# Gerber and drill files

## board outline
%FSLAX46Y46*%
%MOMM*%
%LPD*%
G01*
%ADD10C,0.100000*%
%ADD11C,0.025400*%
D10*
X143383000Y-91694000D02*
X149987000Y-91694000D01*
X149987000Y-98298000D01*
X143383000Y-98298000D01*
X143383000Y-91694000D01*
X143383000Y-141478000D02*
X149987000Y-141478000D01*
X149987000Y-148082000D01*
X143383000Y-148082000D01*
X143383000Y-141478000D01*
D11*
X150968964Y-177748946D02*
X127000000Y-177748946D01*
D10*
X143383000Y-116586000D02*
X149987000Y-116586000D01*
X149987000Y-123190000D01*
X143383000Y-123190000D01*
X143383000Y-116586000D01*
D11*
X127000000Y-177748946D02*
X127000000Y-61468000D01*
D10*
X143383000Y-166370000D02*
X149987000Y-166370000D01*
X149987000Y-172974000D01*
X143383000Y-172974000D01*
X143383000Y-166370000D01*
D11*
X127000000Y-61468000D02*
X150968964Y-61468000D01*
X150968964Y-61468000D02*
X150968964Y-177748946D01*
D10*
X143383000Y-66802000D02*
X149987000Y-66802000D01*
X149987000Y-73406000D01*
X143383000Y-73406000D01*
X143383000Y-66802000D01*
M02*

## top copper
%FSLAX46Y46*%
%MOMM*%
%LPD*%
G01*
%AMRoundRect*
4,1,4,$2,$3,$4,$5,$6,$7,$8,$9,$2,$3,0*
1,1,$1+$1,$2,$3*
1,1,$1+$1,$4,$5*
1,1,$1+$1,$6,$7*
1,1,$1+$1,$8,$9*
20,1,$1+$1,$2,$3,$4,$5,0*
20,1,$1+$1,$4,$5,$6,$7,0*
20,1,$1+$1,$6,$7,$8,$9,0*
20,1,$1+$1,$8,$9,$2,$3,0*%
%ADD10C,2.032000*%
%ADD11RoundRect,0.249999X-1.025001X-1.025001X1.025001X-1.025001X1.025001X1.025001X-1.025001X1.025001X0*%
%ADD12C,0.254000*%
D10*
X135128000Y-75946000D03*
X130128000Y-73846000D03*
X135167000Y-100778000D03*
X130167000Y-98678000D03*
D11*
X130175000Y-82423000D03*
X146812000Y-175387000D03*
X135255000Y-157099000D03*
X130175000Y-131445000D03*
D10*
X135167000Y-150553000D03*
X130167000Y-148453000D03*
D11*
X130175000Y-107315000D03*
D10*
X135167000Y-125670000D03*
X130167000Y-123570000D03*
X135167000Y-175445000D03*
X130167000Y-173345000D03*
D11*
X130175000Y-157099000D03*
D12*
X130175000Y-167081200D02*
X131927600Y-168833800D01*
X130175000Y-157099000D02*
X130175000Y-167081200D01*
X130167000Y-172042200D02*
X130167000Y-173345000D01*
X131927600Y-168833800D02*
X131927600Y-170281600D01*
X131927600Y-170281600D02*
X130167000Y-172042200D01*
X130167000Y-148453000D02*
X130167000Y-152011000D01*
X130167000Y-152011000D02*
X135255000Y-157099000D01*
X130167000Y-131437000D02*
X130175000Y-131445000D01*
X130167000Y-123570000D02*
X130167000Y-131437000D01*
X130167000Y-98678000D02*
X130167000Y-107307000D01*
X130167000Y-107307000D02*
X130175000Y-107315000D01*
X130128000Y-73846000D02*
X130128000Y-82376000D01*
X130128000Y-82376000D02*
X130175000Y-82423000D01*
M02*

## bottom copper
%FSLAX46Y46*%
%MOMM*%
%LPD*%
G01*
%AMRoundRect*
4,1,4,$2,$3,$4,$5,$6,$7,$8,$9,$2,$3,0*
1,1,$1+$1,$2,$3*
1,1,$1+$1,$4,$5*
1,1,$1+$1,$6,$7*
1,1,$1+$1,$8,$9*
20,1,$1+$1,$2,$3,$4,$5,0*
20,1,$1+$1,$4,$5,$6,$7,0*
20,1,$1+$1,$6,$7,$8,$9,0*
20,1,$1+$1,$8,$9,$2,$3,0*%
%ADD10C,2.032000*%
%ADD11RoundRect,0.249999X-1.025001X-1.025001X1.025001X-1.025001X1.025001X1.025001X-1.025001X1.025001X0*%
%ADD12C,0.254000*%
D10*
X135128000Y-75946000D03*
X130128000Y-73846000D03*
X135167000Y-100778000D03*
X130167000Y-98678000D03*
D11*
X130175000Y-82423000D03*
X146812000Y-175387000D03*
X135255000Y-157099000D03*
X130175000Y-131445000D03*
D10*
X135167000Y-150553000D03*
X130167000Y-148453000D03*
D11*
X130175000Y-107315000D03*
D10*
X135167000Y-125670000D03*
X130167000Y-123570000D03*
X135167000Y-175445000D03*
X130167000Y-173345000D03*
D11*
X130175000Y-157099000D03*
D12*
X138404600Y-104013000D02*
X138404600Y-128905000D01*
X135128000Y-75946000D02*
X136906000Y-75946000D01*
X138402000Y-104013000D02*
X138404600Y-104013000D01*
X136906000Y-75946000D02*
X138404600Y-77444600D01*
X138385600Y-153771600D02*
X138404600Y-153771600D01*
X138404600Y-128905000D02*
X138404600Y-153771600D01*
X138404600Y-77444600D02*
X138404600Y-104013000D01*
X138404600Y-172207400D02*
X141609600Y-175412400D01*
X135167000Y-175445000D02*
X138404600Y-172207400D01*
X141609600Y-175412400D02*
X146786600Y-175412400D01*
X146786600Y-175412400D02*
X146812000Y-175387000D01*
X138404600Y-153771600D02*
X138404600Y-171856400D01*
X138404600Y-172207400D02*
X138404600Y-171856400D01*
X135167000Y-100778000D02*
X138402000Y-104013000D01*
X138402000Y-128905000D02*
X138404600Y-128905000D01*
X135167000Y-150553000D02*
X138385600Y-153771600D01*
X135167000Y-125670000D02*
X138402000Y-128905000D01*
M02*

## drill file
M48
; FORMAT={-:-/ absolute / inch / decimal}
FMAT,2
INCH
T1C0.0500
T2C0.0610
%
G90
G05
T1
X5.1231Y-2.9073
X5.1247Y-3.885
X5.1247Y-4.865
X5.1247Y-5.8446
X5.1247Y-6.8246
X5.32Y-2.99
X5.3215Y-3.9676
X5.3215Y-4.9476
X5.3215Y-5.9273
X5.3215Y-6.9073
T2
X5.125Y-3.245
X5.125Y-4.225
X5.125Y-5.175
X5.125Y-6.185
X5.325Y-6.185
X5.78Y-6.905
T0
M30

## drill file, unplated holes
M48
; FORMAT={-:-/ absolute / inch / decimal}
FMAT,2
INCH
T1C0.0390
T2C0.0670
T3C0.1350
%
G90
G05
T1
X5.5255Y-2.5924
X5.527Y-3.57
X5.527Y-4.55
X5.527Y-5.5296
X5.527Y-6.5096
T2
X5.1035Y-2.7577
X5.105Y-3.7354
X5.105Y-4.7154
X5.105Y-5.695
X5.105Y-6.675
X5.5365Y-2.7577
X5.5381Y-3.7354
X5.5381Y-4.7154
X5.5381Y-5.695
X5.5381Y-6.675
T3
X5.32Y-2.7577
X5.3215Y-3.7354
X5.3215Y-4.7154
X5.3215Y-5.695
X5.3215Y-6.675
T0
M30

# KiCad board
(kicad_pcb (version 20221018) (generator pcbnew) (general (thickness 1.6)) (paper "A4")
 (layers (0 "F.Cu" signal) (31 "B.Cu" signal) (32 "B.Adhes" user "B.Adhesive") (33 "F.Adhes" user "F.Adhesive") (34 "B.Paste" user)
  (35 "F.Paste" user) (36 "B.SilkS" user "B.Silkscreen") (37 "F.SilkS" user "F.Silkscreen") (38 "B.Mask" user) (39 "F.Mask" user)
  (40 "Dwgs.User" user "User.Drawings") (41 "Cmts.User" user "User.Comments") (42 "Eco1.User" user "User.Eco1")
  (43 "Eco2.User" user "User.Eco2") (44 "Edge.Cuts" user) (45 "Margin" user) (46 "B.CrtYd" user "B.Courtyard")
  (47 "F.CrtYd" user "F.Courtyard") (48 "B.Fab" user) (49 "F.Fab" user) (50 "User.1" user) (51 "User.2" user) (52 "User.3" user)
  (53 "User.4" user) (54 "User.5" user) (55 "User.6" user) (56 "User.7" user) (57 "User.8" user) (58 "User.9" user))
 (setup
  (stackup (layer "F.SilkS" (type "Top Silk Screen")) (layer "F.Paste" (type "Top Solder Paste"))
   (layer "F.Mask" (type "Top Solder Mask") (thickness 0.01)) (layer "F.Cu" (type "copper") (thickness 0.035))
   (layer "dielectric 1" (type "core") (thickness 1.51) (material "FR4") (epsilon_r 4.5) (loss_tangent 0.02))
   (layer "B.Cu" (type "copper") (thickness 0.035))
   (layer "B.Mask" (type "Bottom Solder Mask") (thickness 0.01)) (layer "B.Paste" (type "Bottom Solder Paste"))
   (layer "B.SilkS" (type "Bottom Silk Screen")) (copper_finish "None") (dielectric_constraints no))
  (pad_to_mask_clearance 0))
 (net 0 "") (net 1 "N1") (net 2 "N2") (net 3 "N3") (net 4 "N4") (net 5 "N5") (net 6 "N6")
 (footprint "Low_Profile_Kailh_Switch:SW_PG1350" (layer "F.Cu") (at 135.128 70.046)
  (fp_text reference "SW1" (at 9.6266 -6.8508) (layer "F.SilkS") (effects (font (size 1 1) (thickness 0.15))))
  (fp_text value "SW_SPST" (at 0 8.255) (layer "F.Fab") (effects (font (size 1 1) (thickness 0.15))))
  (pad "" np_thru_hole circle (at -5.5 0) (size 1.7018 1.7018) (drill 1.7018) (layers "*.Cu" "*.Mask"))
  (pad "" np_thru_hole circle (at 0 0) (size 3.429 3.429) (drill 3.429) (layers "*.Cu" "*.Mask"))
  (pad "" np_thru_hole circle (at 5.22 -4.2) (size 0.9906 0.9906) (drill 0.9906) (layers "*.Cu" "*.Mask"))
  (pad "" np_thru_hole circle (at 5.5 0) (size 1.7018 1.7018) (drill 1.7018) (layers "*.Cu" "*.Mask"))
  (pad "1" thru_hole circle (at 0 5.9) (size 2.032 2.032) (drill 1.27) (layers "*.Cu" "*.Mask") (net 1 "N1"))
  (pad "2" thru_hole circle (at -5 3.8) (size 2.032 2.032) (drill 1.27) (layers "*.Cu" "*.Mask") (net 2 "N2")))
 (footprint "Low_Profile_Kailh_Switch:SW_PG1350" (layer "F.Cu") (at 135.167 94.878)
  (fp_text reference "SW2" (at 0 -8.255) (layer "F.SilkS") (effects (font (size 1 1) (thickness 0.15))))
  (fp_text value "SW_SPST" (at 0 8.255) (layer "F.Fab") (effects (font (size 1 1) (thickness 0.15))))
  (pad "" np_thru_hole circle (at -5.5 0) (size 1.7018 1.7018) (drill 1.7018) (layers "*.Cu" "*.Mask"))
  (pad "" np_thru_hole circle (at 0 0) (size 3.429 3.429) (drill 3.429) (layers "*.Cu" "*.Mask"))
  (pad "" np_thru_hole circle (at 5.22 -4.2) (size 0.9906 0.9906) (drill 0.9906) (layers "*.Cu" "*.Mask"))
  (pad "" np_thru_hole circle (at 5.5 0) (size 1.7018 1.7018) (drill 1.7018) (layers "*.Cu" "*.Mask"))
  (pad "1" thru_hole circle (at 0 5.9) (size 2.032 2.032) (drill 1.27) (layers "*.Cu" "*.Mask") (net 1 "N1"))
  (pad "2" thru_hole circle (at -5 3.8) (size 2.032 2.032) (drill 1.27) (layers "*.Cu" "*.Mask") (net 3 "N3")))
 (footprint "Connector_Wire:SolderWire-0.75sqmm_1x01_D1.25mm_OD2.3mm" (layer "F.Cu") (at 130.175 82.423)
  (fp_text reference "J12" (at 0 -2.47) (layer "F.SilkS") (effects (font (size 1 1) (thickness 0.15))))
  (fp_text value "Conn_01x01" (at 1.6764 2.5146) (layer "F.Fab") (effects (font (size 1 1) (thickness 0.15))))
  (pad "1" thru_hole roundrect (at 0 0) (size 2.55 2.55) (drill 1.55) (layers "*.Cu" "*.Mask") (roundrect_rratio 0.09803882353) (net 2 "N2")))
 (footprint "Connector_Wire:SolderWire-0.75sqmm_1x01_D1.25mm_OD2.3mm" (layer "F.Cu") (at 146.812 175.387)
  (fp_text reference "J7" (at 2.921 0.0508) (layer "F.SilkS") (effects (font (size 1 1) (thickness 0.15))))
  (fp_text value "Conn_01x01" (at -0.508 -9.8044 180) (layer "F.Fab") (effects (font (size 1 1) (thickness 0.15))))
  (pad "1" thru_hole roundrect (at 0 0) (size 2.55 2.55) (drill 1.55) (layers "*.Cu" "*.Mask") (roundrect_rratio 0.09803882353) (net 1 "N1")))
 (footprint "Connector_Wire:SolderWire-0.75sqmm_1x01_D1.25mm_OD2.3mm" (layer "F.Cu") (at 135.255 157.099)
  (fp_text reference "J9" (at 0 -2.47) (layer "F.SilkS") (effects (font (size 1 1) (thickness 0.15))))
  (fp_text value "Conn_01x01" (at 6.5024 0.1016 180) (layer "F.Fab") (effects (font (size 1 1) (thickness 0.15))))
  (pad "1" thru_hole roundrect (at 0 0) (size 2.55 2.55) (drill 1.55) (layers "*.Cu" "*.Mask") (roundrect_rratio 0.09803882353) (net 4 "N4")))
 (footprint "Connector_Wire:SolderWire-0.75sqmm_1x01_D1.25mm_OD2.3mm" (layer "F.Cu") (at 130.175 131.445)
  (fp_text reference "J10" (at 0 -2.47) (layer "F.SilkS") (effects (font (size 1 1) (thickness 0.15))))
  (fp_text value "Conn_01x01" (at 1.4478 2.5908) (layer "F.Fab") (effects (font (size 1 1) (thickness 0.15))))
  (pad "1" thru_hole roundrect (at 0 0) (size 2.55 2.55) (drill 1.55) (layers "*.Cu" "*.Mask") (roundrect_rratio 0.09803882353) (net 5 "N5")))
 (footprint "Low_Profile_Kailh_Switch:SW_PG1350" (layer "F.Cu") (at 135.167 144.653)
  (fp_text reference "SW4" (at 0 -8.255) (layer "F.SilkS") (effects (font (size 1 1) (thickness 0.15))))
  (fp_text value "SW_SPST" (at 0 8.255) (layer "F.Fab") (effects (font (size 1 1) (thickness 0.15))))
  (pad "" np_thru_hole circle (at -5.5 0) (size 1.7018 1.7018) (drill 1.7018) (layers "*.Cu" "*.Mask"))
  (pad "" np_thru_hole circle (at 0 0) (size 3.429 3.429) (drill 3.429) (layers "*.Cu" "*.Mask"))
  (pad "" np_thru_hole circle (at 5.22 -4.2) (size 0.9906 0.9906) (drill 0.9906) (layers "*.Cu" "*.Mask"))
  (pad "" np_thru_hole circle (at 5.5 0) (size 1.7018 1.7018) (drill 1.7018) (layers "*.Cu" "*.Mask"))
  (pad "1" thru_hole circle (at 0 5.9) (size 2.032 2.032) (drill 1.27) (layers "*.Cu" "*.Mask") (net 1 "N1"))
  (pad "2" thru_hole circle (at -5 3.8) (size 2.032 2.032) (drill 1.27) (layers "*.Cu" "*.Mask") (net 4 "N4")))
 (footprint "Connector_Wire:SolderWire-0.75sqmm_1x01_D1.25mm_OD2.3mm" (layer "F.Cu") (at 130.175 107.315)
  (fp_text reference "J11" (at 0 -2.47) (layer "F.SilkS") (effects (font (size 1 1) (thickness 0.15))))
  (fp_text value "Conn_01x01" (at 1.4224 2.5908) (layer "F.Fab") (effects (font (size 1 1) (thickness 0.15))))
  (pad "1" thru_hole roundrect (at 0 0) (size 2.55 2.55) (drill 1.55) (layers "*.Cu" "*.Mask") (roundrect_rratio 0.09803882353) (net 3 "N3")))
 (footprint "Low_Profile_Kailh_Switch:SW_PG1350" (layer "F.Cu") (at 135.167 119.77)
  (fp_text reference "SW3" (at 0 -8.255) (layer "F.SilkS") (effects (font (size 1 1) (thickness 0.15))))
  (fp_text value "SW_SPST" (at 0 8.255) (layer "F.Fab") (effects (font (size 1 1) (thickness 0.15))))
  (pad "" np_thru_hole circle (at -5.5 0) (size 1.7018 1.7018) (drill 1.7018) (layers "*.Cu" "*.Mask"))
  (pad "" np_thru_hole circle (at 0 0) (size 3.429 3.429) (drill 3.429) (layers "*.Cu" "*.Mask"))
  (pad "" np_thru_hole circle (at 5.22 -4.2) (size 0.9906 0.9906) (drill 0.9906) (layers "*.Cu" "*.Mask"))
  (pad "" np_thru_hole circle (at 5.5 0) (size 1.7018 1.7018) (drill 1.7018) (layers "*.Cu" "*.Mask"))
  (pad "1" thru_hole circle (at 0 5.9) (size 2.032 2.032) (drill 1.27) (layers "*.Cu" "*.Mask") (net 1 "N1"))
  (pad "2" thru_hole circle (at -5 3.8) (size 2.032 2.032) (drill 1.27) (layers "*.Cu" "*.Mask") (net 5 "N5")))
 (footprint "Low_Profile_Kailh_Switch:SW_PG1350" (layer "F.Cu") (at 135.167 169.545)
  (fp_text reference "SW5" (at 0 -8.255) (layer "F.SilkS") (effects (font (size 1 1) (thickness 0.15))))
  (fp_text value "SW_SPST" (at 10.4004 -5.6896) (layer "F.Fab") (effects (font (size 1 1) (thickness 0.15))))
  (pad "" np_thru_hole circle (at -5.5 0) (size 1.7018 1.7018) (drill 1.7018) (layers "*.Cu" "*.Mask"))
  (pad "" np_thru_hole circle (at 0 0) (size 3.429 3.429) (drill 3.429) (layers "*.Cu" "*.Mask"))
  (pad "" np_thru_hole circle (at 5.22 -4.2) (size 0.9906 0.9906) (drill 0.9906) (layers "*.Cu" "*.Mask"))
  (pad "" np_thru_hole circle (at 5.5 0) (size 1.7018 1.7018) (drill 1.7018) (layers "*.Cu" "*.Mask"))
  (pad "1" thru_hole circle (at 0 5.9) (size 2.032 2.032) (drill 1.27) (layers "*.Cu" "*.Mask") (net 1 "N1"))
  (pad "2" thru_hole circle (at -5 3.8) (size 2.032 2.032) (drill 1.27) (layers "*.Cu" "*.Mask") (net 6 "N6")))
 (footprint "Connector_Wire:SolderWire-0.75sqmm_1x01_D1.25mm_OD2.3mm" (layer "F.Cu") (at 130.175 157.099)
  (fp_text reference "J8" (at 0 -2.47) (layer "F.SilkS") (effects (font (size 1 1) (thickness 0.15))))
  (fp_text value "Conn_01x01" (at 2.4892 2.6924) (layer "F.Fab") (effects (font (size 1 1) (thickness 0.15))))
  (pad "1" thru_hole roundrect (at 0 0) (size 2.55 2.55) (drill 1.55) (layers "*.Cu" "*.Mask") (roundrect_rratio 0.09803882353) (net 6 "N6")))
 (gr_rect (start 143.383 91.694) (end 149.987 98.298) (stroke (width 0.1) (type default)) (fill none) (layer "Edge.Cuts"))
 (gr_rect (start 143.383 141.478) (end 149.987 148.082) (stroke (width 0.1) (type default)) (fill none) (layer "Edge.Cuts"))
 (gr_line (start 150.968964 177.748946) (end 127 177.748946) (stroke (width 0.0254) (type default)) (layer "Edge.Cuts"))
 (gr_rect (start 143.383 116.586) (end 149.987 123.19) (stroke (width 0.1) (type default)) (fill none) (layer "Edge.Cuts"))
 (gr_line (start 127 177.748946) (end 127 61.468) (stroke (width 0.0254) (type default)) (layer "Edge.Cuts"))
 (gr_rect (start 143.383 166.37) (end 149.987 172.974) (stroke (width 0.1) (type default)) (fill none) (layer "Edge.Cuts"))
 (gr_line (start 127 61.468) (end 150.968964 61.468) (stroke (width 0.0254) (type default)) (layer "Edge.Cuts"))
 (gr_line (start 150.968964 61.468) (end 150.968964 177.748946) (stroke (width 0.0254) (type default)) (layer "Edge.Cuts"))
 (gr_rect (start 143.383 66.802) (end 149.987 73.406) (stroke (width 0.1) (type default)) (fill none) (layer "Edge.Cuts"))
 (segment (start 138.4046 104.013) (end 138.4046 128.905) (width 0.254) (layer "B.Cu") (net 1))
 (segment (start 135.128 75.946) (end 136.906 75.946) (width 0.254) (layer "B.Cu") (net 1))
 (segment (start 138.402 104.013) (end 138.4046 104.013) (width 0.254) (layer "B.Cu") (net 1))
 (segment (start 136.906 75.946) (end 138.4046 77.4446) (width 0.254) (layer "B.Cu") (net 1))
 (segment (start 138.3856 153.7716) (end 138.4046 153.7716) (width 0.254) (layer "B.Cu") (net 1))
 (segment (start 138.4046 128.905) (end 138.4046 153.7716) (width 0.254) (layer "B.Cu") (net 1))
 (segment (start 138.4046 77.4446) (end 138.4046 104.013) (width 0.254) (layer "B.Cu") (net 1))
 (segment (start 138.4046 172.2074) (end 141.6096 175.4124) (width 0.254) (layer "B.Cu") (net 1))
 (segment (start 135.167 175.445) (end 138.4046 172.2074) (width 0.254) (layer "B.Cu") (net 1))
 (segment (start 141.6096 175.4124) (end 146.7866 175.4124) (width 0.254) (layer "B.Cu") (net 1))
 (segment (start 146.7866 175.4124) (end 146.812 175.387) (width 0.254) (layer "B.Cu") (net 1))
 (segment (start 138.4046 153.7716) (end 138.4046 171.8564) (width 0.254) (layer "B.Cu") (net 1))
 (segment (start 138.4046 172.2074) (end 138.4046 171.8564) (width 0.254) (layer "B.Cu") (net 1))
 (segment (start 135.167 100.778) (end 138.402 104.013) (width 0.254) (layer "B.Cu") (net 1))
 (segment (start 138.402 128.905) (end 138.4046 128.905) (width 0.254) (layer "B.Cu") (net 1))
 (segment (start 135.167 150.553) (end 138.3856 153.7716) (width 0.254) (layer "B.Cu") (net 1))
 (segment (start 135.167 125.67) (end 138.402 128.905) (width 0.254) (layer "B.Cu") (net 1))
 (segment (start 130.175 167.0812) (end 131.9276 168.8338) (width 0.254) (layer "F.Cu") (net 6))
 (segment (start 130.175 157.099) (end 130.175 167.0812) (width 0.254) (layer "F.Cu") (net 6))
 (segment (start 130.167 172.0422) (end 130.167 173.345) (width 0.254) (layer "F.Cu") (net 6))
 (segment (start 131.9276 168.8338) (end 131.9276 170.2816) (width 0.254) (layer "F.Cu") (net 6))
 (segment (start 131.9276 170.2816) (end 130.167 172.0422) (width 0.254) (layer "F.Cu") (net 6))
 (segment (start 130.167 148.453) (end 130.167 152.011) (width 0.254) (layer "F.Cu") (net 4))
 (segment (start 130.167 152.011) (end 135.255 157.099) (width 0.254) (layer "F.Cu") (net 4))
 (segment (start 130.167 131.437) (end 130.175 131.445) (width 0.254) (layer "F.Cu") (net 5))
 (segment (start 130.167 123.57) (end 130.167 131.437) (width 0.254) (layer "F.Cu") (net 5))
 (segment (start 130.167 98.678) (end 130.167 107.307) (width 0.254) (layer "F.Cu") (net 3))
 (segment (start 130.167 107.307) (end 130.175 107.315) (width 0.254) (layer "F.Cu") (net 3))
 (segment (start 130.128 73.846) (end 130.128 82.376) (width 0.254) (layer "F.Cu") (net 2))
 (segment (start 130.128 82.376) (end 130.175 82.423) (width 0.254) (layer "F.Cu") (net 2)))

